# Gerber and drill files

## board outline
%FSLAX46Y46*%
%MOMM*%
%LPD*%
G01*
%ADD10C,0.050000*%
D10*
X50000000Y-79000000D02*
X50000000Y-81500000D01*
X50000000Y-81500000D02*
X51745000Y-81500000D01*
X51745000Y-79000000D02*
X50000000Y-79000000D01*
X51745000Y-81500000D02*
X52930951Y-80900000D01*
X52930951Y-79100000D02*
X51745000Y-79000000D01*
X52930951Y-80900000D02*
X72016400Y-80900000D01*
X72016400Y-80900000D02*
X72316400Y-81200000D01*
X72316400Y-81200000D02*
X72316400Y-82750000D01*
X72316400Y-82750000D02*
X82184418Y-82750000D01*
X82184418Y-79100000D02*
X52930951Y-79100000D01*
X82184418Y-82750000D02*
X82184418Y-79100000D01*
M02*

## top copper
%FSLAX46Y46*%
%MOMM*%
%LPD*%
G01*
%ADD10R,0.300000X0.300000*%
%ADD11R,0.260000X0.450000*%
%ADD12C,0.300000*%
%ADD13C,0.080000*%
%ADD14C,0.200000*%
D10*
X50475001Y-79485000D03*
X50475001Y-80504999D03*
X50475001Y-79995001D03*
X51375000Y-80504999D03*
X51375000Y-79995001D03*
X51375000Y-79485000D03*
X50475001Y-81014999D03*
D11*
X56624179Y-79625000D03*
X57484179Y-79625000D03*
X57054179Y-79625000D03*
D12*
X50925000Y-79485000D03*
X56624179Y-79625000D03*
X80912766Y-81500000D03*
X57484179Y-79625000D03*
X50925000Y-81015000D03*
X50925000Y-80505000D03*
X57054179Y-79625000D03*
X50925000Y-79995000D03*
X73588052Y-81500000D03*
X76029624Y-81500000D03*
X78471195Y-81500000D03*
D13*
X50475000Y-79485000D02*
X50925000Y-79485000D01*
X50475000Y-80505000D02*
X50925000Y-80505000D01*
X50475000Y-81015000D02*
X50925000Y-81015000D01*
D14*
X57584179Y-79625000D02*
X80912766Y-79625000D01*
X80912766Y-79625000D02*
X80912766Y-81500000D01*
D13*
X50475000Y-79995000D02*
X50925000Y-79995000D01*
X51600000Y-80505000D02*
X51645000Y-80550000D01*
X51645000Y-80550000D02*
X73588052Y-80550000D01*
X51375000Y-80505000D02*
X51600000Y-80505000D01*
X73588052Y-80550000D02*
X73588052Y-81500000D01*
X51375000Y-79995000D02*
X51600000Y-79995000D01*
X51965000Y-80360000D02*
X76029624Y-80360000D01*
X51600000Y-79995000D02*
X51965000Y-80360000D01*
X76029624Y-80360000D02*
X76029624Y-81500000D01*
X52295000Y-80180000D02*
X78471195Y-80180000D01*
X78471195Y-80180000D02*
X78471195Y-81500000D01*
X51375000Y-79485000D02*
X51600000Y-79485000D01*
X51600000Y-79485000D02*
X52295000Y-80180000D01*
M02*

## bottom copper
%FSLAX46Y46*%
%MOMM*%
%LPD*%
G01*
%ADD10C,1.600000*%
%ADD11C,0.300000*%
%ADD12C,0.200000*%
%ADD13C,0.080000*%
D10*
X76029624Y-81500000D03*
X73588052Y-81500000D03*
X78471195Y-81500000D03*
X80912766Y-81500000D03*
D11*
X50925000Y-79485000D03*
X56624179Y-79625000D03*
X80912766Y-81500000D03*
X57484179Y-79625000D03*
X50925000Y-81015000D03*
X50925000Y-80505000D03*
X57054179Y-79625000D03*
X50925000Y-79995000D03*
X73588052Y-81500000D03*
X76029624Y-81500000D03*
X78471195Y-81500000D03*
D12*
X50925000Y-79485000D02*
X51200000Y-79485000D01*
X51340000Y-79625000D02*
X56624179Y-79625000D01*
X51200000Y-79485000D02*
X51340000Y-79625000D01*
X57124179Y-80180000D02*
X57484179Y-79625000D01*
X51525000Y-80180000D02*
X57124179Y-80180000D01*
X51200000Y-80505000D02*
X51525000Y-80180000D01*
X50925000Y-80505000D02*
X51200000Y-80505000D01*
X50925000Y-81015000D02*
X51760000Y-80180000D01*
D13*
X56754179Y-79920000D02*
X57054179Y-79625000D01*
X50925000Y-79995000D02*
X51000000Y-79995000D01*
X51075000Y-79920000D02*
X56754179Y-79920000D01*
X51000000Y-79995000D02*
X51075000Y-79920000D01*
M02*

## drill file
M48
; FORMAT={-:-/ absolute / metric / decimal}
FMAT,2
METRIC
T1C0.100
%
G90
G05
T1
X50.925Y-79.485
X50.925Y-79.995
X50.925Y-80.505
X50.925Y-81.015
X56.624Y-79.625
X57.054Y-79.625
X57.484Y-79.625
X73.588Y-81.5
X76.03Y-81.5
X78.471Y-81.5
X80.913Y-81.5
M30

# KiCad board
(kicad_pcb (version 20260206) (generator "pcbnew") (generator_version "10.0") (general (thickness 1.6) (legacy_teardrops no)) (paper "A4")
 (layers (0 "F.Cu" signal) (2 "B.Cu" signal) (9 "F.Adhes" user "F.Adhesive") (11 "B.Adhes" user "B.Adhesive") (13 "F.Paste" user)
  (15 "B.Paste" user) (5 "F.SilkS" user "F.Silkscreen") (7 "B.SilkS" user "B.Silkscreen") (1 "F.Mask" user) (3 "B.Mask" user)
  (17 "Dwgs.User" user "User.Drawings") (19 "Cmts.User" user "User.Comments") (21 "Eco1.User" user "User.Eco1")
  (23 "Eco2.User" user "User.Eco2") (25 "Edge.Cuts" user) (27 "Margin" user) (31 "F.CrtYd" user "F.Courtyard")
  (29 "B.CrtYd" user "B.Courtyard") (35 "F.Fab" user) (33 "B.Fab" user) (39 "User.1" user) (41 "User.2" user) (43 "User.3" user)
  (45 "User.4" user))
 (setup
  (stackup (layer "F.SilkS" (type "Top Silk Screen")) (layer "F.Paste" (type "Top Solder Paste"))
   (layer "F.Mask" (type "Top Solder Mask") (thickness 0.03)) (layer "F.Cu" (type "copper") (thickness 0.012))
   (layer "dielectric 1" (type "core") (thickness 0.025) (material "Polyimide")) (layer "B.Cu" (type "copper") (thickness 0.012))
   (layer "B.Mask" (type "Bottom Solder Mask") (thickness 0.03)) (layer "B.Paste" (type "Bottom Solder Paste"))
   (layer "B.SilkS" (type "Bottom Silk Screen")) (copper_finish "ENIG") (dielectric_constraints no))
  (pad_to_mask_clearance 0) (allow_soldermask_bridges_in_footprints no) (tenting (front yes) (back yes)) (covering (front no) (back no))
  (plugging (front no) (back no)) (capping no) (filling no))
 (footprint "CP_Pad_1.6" (layer "F.Cu") (at 78.471195 81.5)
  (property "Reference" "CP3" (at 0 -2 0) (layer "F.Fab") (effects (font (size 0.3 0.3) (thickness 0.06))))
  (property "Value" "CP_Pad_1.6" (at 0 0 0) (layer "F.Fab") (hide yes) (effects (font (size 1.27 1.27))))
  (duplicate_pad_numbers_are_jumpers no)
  (pad "1" smd circle (at 0 0) (size 1.6 1.6) (layers "B.Cu" "B.Mask") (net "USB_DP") (solder_mask_margin 0.1)))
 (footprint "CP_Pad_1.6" (layer "F.Cu") (at 76.029624 81.5)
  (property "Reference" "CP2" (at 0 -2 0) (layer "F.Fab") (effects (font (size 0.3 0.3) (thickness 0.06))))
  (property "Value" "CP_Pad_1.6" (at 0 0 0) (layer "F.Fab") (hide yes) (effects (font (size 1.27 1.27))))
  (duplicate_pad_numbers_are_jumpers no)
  (pad "1" smd circle (at 0 0) (size 1.6 1.6) (layers "B.Cu" "B.Mask") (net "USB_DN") (solder_mask_margin 0.1)))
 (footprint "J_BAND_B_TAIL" (layer "F.Cu") (at 50.9 80.25)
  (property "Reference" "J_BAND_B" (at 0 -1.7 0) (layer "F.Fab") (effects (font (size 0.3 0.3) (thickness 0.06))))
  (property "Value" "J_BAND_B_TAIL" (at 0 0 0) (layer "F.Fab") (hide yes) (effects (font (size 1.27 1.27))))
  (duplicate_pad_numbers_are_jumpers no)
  (pad "1" smd rect (at -0.424999 -0.765) (size 0.3 0.3) (layers "F.Cu" "F.Mask") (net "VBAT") (solder_mask_margin 0.05)
   (thermal_bridge_angle 45))
  (pad "2" smd rect (at -0.424999 0.254999) (size 0.3 0.3) (layers "F.Cu" "F.Mask") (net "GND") (solder_mask_margin 0.05)
   (thermal_bridge_angle 45))
  (pad "3" smd rect (at -0.424999 -0.254999) (size 0.3 0.3) (layers "F.Cu" "F.Mask") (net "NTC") (solder_mask_margin 0.05)
   (thermal_bridge_angle 45))
  (pad "4" smd rect (at 0.475 0.254999) (size 0.3 0.3) (layers "F.Cu" "F.Mask") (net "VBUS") (solder_mask_margin 0.05)
   (thermal_bridge_angle 45))
  (pad "5" smd rect (at 0.475 -0.254999) (size 0.3 0.3) (layers "F.Cu" "F.Mask") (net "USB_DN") (solder_mask_margin 0.05)
   (thermal_bridge_angle 45))
  (pad "6" smd rect (at 0.475 -0.765) (size 0.3 0.3) (layers "F.Cu" "F.Mask") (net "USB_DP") (solder_mask_margin 0.05)
   (thermal_bridge_angle 45))
  (pad "7" smd rect (at -0.424999 0.764999) (size 0.3 0.3) (layers "F.Cu" "F.Mask") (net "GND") (solder_mask_margin 0.05)
   (thermal_bridge_angle 45)))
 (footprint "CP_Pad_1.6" (layer "F.Cu") (at 80.912766 81.5)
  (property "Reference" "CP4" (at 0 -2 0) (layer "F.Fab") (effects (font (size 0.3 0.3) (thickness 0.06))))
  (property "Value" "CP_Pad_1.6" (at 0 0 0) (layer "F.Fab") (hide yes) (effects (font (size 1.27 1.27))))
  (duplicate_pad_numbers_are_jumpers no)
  (pad "1" smd circle (at 0 0) (size 1.6 1.6) (layers "B.Cu" "B.Mask") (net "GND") (solder_mask_margin 0.1)))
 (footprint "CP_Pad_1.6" (layer "F.Cu") (at 73.588052 81.5)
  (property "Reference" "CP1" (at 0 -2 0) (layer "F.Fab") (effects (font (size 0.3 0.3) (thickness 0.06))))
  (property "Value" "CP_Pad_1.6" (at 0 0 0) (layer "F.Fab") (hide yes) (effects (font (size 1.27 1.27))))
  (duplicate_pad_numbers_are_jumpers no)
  (pad "1" smd circle (at 0 0) (size 1.6 1.6) (layers "B.Cu" "B.Mask") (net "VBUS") (solder_mask_margin 0.1)))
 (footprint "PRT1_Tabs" (layer "F.Cu") (at 57.054179 79.625)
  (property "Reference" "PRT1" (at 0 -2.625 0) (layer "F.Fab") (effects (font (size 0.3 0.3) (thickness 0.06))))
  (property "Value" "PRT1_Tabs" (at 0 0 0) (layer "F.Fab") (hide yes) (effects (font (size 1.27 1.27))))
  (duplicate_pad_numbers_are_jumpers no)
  (pad "1" smd rect (at -0.43 0) (size 0.26 0.45) (layers "F.Cu" "F.Mask") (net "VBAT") (solder_mask_margin 0.05) (thermal_bridge_angle 45))
  (pad "2" smd rect (at 0.43 0) (size 0.26 0.45) (layers "F.Cu" "F.Mask") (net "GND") (solder_mask_margin 0.05) (thermal_bridge_angle 45))
  (pad "3" smd rect (at 0 0) (size 0.26 0.45) (layers "F.Cu" "F.Mask") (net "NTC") (solder_mask_margin 0.05) (thermal_bridge_angle 45)))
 (gr_line (start 50 79) (end 50 81.5) (stroke (width 0.05) (type default)) (layer "Edge.Cuts"))
 (gr_line (start 50 81.5) (end 51.745 81.5) (stroke (width 0.05) (type default)) (layer "Edge.Cuts"))
 (gr_line (start 51.745 79) (end 50 79) (stroke (width 0.05) (type default)) (layer "Edge.Cuts"))
 (gr_line (start 51.745 81.5) (end 52.930951 80.9) (stroke (width 0.05) (type default)) (layer "Edge.Cuts"))
 (gr_line (start 52.930951 79.1) (end 51.745 79) (stroke (width 0.05) (type default)) (layer "Edge.Cuts"))
 (gr_line (start 52.930951 80.9) (end 72.0164 80.9) (stroke (width 0.05) (type default)) (layer "Edge.Cuts"))
 (gr_line (start 72.0164 80.9) (end 72.3164 81.2) (stroke (width 0.05) (type default)) (layer "Edge.Cuts"))
 (gr_line (start 72.3164 81.2) (end 72.3164 82.75) (stroke (width 0.05) (type default)) (layer "Edge.Cuts"))
 (gr_line (start 72.3164 82.75) (end 82.184418 82.75) (stroke (width 0.05) (type default)) (layer "Edge.Cuts"))
 (gr_line (start 82.184418 79.1) (end 52.930951 79.1) (stroke (width 0.05) (type default)) (layer "Edge.Cuts"))
 (gr_line (start 82.184418 82.75) (end 82.184418 79.1) (stroke (width 0.05) (type default)) (layer "Edge.Cuts"))
 (segment (start 50.475 79.485) (end 50.925 79.485) (width 0.08) (layer "F.Cu") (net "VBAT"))
 (via (at 50.925 79.485) (size 0.3) (drill 0.1) (layers "F.Cu" "B.Cu") (tenting (front yes) (back yes)) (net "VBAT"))
 (via (at 56.624179 79.625) (size 0.3) (drill 0.1) (layers "F.Cu" "B.Cu") (tenting (front yes) (back yes)) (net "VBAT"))
 (segment (start 51.34 79.625) (end 56.624179 79.625) (width 0.2) (layer "B.Cu") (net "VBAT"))
 (segment (start 51.2 79.485) (end 51.34 79.625) (width 0.2) (layer "B.Cu") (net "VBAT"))
 (segment (start 50.925 79.485) (end 51.2 79.485) (width 0.2) (layer "B.Cu") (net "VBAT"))
 (segment (start 50.475 81.015) (end 50.925 81.015) (width 0.08) (layer "F.Cu") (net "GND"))
 (segment (start 57.584179 79.625) (end 80.912766 79.625) (width 0.2) (layer "F.Cu") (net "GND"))
 (segment (start 50.475 80.505) (end 50.925 80.505) (width 0.08) (layer "F.Cu") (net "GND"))
 (segment (start 80.912766 79.625) (end 80.912766 81.5) (width 0.2) (layer "F.Cu") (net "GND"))
 (via (at 50.925 81.015) (size 0.3) (drill 0.1) (layers "F.Cu" "B.Cu") (tenting (front yes) (back yes)) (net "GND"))
 (via (at 50.925 80.505) (size 0.3) (drill 0.1) (layers "F.Cu" "B.Cu") (tenting (front yes) (back yes)) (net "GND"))
 (via (at 57.484179 79.625) (size 0.3) (drill 0.1) (layers "F.Cu" "B.Cu") (tenting (front yes) (back yes)) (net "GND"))
 (via (at 80.912766 81.5) (size 0.3) (drill 0.1) (layers "F.Cu" "B.Cu") (tenting (front yes) (back yes)) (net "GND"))
 (segment (start 50.925 80.505) (end 51.2 80.505) (width 0.2) (layer "B.Cu") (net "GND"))
 (segment (start 51.525 80.18) (end 57.124179 80.18) (width 0.2) (layer "B.Cu") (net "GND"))
 (segment (start 50.925 81.015) (end 51.76 80.18) (width 0.2) (layer "B.Cu") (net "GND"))
 (segment (start 51.2 80.505) (end 51.525 80.18) (width 0.2) (layer "B.Cu") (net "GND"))
 (segment (start 57.124179 80.18) (end 57.484179 79.625) (width 0.2) (layer "B.Cu") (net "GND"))
 (segment (start 50.475 79.995) (end 50.925 79.995) (width 0.08) (layer "F.Cu") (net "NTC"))
 (via (at 57.054179 79.625) (size 0.3) (drill 0.1) (layers "F.Cu" "B.Cu") (tenting (front yes) (back yes)) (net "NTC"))
 (via (at 50.925 79.995) (size 0.3) (drill 0.1) (layers "F.Cu" "B.Cu") (tenting (front yes) (back yes)) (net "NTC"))
 (segment (start 56.754179 79.92) (end 57.054179 79.625) (width 0.08) (layer "B.Cu") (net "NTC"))
 (segment (start 51.075 79.92) (end 56.754179 79.92) (width 0.08) (layer "B.Cu") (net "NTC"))
 (segment (start 50.925 79.995) (end 51 79.995) (width 0.08) (layer "B.Cu") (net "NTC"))
 (segment (start 51 79.995) (end 51.075 79.92) (width 0.08) (layer "B.Cu") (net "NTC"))
 (segment (start 51.6 80.505) (end 51.645 80.55) (width 0.08) (layer "F.Cu") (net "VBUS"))
 (segment (start 73.588052 80.55) (end 73.588052 81.5) (width 0.08) (layer "F.Cu") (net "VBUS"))
 (segment (start 51.645 80.55) (end 73.588052 80.55) (width 0.08) (layer "F.Cu") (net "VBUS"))
 (segment (start 51.375 80.505) (end 51.6 80.505) (width 0.08) (layer "F.Cu") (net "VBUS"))
 (via (at 73.588052 81.5) (size 0.3) (drill 0.1) (layers "F.Cu" "B.Cu") (tenting (front yes) (back yes)) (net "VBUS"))
 (segment (start 51.6 79.995) (end 51.965 80.36) (width 0.08) (layer "F.Cu") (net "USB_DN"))
 (segment (start 51.965 80.36) (end 76.029624 80.36) (width 0.08) (layer "F.Cu") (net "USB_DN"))
 (segment (start 51.375 79.995) (end 51.6 79.995) (width 0.08) (layer "F.Cu") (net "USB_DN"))
 (segment (start 76.029624 80.36) (end 76.029624 81.5) (width 0.08) (layer "F.Cu") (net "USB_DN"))
 (via (at 76.029624 81.5) (size 0.3) (drill 0.1) (layers "F.Cu" "B.Cu") (tenting (front yes) (back yes)) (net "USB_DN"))
 (segment (start 52.295 80.18) (end 78.471195 80.18) (width 0.08) (layer "F.Cu") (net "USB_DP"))
 (segment (start 78.471195 80.18) (end 78.471195 81.5) (width 0.08) (layer "F.Cu") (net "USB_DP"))
 (segment (start 51.375 79.485) (end 51.6 79.485) (width 0.08) (layer "F.Cu") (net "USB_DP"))
 (segment (start 51.6 79.485) (end 52.295 80.18) (width 0.08) (layer "F.Cu") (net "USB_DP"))
 (via (at 78.471195 81.5) (size 0.3) (drill 0.1) (layers "F.Cu" "B.Cu") (tenting (front yes) (back yes)) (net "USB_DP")))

